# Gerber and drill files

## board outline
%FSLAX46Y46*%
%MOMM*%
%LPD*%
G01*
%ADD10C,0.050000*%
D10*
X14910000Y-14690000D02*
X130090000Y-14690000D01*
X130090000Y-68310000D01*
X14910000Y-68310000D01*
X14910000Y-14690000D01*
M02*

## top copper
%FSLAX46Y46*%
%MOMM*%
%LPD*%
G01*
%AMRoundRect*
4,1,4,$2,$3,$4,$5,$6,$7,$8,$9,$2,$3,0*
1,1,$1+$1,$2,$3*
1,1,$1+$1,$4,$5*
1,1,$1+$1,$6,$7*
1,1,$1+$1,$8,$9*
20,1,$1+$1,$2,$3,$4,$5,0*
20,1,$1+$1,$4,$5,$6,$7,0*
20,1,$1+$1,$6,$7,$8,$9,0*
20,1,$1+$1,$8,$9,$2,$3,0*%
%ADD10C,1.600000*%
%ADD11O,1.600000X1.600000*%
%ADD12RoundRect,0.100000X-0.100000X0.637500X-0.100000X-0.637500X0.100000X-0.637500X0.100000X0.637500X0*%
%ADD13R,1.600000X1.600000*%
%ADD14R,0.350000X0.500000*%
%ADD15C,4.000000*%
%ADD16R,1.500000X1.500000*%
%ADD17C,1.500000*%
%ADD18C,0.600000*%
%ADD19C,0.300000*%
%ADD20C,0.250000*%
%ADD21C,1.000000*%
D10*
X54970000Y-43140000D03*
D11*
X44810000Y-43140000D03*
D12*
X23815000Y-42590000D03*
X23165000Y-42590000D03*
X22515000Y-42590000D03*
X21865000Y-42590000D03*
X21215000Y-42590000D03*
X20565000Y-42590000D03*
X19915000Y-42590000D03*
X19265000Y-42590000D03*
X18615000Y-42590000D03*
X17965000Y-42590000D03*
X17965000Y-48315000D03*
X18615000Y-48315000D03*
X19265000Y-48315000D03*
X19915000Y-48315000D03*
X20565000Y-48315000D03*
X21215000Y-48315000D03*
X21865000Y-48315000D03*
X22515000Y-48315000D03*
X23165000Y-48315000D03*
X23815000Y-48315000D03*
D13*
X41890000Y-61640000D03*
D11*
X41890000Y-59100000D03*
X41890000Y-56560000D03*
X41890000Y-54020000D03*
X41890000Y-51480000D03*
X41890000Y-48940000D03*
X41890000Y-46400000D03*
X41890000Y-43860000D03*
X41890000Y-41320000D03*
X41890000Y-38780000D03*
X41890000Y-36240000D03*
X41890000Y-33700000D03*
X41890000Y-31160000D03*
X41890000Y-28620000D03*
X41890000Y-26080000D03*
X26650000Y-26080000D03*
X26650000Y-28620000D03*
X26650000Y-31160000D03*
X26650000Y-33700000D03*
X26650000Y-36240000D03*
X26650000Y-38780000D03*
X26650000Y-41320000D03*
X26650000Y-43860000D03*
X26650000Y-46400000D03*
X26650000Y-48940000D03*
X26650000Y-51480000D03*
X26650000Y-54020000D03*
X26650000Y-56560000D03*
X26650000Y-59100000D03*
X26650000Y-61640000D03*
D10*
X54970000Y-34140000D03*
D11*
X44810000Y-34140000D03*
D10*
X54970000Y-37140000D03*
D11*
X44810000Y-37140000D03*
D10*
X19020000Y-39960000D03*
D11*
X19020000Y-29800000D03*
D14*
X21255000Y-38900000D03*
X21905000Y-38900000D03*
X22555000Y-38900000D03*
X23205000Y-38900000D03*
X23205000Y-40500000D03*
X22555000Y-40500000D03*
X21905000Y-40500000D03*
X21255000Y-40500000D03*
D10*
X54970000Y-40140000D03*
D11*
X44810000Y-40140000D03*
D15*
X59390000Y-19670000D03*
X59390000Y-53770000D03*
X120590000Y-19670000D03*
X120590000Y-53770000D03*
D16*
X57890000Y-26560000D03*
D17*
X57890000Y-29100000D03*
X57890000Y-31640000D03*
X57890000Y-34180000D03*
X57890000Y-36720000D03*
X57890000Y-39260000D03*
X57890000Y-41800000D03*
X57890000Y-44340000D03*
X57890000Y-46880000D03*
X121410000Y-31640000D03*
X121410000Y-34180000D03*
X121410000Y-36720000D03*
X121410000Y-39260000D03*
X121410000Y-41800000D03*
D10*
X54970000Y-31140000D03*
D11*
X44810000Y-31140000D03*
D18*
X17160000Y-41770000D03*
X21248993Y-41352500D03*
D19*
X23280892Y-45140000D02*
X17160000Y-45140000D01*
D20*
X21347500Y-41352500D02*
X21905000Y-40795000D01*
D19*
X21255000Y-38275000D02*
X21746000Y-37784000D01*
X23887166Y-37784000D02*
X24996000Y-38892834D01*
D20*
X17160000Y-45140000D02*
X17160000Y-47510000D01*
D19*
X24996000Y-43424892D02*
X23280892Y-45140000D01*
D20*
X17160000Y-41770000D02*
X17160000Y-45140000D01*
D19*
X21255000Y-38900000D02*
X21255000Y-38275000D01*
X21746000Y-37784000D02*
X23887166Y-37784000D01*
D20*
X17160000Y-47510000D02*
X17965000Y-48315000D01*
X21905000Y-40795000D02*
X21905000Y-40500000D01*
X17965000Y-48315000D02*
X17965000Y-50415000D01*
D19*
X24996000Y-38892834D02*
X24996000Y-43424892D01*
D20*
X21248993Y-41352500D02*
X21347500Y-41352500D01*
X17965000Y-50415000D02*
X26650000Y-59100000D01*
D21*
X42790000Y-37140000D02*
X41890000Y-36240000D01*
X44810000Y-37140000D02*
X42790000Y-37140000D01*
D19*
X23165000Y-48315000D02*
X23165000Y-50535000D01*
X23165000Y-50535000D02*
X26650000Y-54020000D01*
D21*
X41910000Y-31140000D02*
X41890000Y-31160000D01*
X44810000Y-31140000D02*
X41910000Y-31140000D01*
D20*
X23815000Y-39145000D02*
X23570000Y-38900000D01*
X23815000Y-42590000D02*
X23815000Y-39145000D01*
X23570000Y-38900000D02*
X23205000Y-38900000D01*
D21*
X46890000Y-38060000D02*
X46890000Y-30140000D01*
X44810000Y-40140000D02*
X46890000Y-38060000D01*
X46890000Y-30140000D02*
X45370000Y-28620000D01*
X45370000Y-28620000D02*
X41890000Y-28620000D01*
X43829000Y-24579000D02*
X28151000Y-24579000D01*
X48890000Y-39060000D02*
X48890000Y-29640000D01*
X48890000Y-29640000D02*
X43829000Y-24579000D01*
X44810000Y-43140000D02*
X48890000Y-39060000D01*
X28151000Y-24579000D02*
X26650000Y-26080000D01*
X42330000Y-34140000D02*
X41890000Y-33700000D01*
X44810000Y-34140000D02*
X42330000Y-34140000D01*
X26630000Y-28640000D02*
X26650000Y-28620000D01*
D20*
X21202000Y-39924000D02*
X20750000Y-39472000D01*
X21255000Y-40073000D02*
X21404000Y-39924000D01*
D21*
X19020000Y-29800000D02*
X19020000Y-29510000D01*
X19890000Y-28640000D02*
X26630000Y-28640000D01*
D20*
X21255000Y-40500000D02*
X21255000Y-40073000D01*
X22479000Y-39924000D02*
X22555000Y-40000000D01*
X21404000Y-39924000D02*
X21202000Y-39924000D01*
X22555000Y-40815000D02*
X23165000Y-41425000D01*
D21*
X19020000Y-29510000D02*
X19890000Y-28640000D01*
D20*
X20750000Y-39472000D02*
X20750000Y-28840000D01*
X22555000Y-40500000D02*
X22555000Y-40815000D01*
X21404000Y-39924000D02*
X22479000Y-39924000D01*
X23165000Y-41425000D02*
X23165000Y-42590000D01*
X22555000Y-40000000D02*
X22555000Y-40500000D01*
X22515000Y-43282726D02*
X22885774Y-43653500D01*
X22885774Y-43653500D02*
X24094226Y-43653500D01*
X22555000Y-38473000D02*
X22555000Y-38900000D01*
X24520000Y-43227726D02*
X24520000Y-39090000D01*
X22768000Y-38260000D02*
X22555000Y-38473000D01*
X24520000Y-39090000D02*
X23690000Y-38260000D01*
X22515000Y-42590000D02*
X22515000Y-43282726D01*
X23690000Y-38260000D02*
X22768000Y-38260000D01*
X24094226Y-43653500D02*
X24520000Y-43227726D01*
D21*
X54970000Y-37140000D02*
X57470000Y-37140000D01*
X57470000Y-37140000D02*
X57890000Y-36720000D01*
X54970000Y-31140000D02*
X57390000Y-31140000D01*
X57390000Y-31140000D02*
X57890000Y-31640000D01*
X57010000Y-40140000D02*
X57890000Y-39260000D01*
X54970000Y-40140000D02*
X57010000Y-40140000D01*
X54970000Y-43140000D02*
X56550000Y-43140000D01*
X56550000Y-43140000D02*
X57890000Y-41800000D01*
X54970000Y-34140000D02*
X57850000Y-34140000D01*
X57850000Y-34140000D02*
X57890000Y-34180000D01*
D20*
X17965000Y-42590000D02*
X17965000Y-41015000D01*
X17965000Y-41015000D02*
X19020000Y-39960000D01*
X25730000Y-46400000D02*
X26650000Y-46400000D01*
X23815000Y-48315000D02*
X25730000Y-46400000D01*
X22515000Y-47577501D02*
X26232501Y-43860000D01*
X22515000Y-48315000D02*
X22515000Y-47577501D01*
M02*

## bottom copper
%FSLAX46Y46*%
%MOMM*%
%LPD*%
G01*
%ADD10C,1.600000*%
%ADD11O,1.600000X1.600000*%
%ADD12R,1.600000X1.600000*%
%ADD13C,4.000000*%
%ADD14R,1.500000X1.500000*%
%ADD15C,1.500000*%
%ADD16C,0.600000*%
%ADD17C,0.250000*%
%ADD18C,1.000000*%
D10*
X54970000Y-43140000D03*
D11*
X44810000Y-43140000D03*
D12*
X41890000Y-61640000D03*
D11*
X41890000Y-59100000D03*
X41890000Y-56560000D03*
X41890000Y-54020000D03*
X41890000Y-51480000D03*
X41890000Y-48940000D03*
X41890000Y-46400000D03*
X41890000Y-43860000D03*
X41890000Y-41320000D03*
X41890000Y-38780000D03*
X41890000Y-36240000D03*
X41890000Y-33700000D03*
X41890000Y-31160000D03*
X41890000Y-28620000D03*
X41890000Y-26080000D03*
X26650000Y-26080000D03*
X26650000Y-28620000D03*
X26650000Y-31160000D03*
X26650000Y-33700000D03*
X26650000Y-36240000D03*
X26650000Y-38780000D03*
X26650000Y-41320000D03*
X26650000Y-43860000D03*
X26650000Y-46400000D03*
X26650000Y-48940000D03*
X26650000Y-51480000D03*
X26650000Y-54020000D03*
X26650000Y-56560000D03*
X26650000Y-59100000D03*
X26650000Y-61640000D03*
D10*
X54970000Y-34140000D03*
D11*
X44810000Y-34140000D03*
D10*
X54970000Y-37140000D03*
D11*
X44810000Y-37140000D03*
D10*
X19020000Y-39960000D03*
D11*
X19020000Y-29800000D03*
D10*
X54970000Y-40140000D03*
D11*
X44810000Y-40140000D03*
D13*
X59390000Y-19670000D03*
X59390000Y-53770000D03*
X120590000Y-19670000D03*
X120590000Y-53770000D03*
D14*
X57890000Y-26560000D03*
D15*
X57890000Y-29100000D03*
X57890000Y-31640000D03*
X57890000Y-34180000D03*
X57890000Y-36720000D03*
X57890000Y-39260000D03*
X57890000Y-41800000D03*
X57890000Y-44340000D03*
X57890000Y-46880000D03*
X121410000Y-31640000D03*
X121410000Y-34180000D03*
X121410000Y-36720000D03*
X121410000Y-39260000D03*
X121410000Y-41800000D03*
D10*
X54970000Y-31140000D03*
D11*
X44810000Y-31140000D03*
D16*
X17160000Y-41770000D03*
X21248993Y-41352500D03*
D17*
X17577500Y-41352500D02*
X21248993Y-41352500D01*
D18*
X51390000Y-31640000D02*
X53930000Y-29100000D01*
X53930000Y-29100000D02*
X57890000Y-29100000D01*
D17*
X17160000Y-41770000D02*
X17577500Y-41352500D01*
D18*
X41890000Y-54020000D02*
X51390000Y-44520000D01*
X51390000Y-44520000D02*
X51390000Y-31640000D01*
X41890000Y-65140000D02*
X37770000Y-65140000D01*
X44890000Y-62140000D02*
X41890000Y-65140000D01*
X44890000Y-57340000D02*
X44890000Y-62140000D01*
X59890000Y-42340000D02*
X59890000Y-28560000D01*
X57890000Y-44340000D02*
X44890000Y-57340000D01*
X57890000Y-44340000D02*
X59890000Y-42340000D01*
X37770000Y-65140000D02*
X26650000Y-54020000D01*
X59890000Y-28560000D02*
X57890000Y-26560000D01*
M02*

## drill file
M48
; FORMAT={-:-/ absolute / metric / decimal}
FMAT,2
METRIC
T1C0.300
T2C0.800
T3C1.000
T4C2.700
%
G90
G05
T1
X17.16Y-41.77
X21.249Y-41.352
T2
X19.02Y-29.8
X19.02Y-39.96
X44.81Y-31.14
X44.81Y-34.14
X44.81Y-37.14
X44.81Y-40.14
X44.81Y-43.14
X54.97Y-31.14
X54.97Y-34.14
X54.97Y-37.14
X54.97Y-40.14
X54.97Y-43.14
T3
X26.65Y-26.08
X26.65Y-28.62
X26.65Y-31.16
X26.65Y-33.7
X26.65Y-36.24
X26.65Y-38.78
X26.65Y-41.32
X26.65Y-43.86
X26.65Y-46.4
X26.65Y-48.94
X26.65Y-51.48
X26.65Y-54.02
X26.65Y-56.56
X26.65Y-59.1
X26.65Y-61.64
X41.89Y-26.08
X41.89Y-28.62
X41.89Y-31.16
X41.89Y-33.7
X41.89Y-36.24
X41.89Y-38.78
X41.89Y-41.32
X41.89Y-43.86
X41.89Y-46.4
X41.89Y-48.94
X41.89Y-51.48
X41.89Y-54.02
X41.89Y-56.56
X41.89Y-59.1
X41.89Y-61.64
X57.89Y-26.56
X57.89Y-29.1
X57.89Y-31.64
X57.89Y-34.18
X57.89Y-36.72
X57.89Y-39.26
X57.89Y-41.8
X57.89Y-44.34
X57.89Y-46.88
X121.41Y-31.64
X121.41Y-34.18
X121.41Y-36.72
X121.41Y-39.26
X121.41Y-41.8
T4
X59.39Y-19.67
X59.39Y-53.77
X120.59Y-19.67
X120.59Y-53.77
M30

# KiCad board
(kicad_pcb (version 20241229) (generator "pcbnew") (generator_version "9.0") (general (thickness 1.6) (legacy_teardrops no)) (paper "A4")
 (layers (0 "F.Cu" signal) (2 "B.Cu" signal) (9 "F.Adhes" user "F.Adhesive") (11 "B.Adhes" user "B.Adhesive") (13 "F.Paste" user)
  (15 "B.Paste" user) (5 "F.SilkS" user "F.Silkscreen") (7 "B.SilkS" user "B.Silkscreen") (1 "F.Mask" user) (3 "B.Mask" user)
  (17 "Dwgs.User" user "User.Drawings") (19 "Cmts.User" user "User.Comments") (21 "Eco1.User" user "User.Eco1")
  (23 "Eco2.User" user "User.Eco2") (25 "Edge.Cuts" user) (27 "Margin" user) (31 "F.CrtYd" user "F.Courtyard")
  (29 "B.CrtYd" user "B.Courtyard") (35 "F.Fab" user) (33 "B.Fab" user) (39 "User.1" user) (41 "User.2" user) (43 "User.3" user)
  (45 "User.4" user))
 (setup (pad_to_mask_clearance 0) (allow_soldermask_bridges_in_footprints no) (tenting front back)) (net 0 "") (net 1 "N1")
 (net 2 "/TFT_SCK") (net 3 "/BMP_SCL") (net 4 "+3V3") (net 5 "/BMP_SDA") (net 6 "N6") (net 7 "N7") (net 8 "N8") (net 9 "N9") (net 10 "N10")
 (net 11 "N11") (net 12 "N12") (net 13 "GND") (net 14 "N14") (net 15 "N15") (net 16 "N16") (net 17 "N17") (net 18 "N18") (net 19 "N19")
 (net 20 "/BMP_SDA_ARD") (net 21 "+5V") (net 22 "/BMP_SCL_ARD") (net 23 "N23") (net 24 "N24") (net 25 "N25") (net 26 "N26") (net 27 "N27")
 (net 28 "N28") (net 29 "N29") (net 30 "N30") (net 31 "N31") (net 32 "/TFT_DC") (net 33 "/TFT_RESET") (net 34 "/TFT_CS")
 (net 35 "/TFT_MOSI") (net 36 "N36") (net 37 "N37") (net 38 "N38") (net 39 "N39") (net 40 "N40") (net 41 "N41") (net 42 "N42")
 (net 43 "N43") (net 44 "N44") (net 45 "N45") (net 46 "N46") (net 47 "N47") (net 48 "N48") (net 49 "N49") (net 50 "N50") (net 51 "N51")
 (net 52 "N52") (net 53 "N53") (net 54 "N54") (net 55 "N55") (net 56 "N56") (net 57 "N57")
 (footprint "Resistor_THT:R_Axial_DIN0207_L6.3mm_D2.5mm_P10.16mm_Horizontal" (layer "F.Cu") (at 54.97 43.14 180)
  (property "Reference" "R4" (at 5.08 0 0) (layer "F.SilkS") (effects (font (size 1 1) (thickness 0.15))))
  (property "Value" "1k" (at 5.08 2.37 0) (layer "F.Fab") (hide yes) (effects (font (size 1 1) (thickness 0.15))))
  (pad "1" thru_hole circle (at 0 0 180) (size 1.6 1.6) (drill 0.8) (layers "*.Cu" "*.Mask") (remove_unused_layers no) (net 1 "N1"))
  (pad "2" thru_hole oval (at 10.16 0 180) (size 1.6 1.6) (drill 0.8) (layers "*.Cu" "*.Mask") (remove_unused_layers no) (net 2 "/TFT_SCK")))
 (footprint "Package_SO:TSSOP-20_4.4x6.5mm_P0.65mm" (layer "F.Cu") (at 20.89 45.4525 -90)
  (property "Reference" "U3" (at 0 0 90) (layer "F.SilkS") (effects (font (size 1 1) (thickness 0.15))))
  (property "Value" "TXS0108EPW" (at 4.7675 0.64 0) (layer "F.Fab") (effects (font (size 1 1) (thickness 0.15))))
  (pad "1" smd roundrect (at -2.8625 -2.925 270) (size 1.475 0.4) (layers "F.Cu" "F.Mask" "F.Paste") (roundrect_rratio 0.25)
   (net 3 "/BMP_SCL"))
  (pad "2" smd roundrect (at -2.8625 -2.275 270) (size 1.475 0.4) (layers "F.Cu" "F.Mask" "F.Paste") (roundrect_rratio 0.25) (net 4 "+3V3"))
  (pad "3" smd roundrect (at -2.8625 -1.625 270) (size 1.475 0.4) (layers "F.Cu" "F.Mask" "F.Paste") (roundrect_rratio 0.25)
   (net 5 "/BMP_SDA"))
  (pad "4" smd roundrect (at -2.8625 -0.975 270) (size 1.475 0.4) (layers "F.Cu" "F.Mask" "F.Paste") (roundrect_rratio 0.25) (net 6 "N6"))
  (pad "5" smd roundrect (at -2.8625 -0.325 270) (size 1.475 0.4) (layers "F.Cu" "F.Mask" "F.Paste") (roundrect_rratio 0.25) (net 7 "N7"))
  (pad "6" smd roundrect (at -2.8625 0.325 270) (size 1.475 0.4) (layers "F.Cu" "F.Mask" "F.Paste") (roundrect_rratio 0.25) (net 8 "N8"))
  (pad "7" smd roundrect (at -2.8625 0.975 270) (size 1.475 0.4) (layers "F.Cu" "F.Mask" "F.Paste") (roundrect_rratio 0.25) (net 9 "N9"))
  (pad "8" smd roundrect (at -2.8625 1.625 270) (size 1.475 0.4) (layers "F.Cu" "F.Mask" "F.Paste") (roundrect_rratio 0.25) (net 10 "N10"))
  (pad "9" smd roundrect (at -2.8625 2.275 270) (size 1.475 0.4) (layers "F.Cu" "F.Mask" "F.Paste") (roundrect_rratio 0.25) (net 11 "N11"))
  (pad "10" smd roundrect (at -2.8625 2.925 270) (size 1.475 0.4) (layers "F.Cu" "F.Mask" "F.Paste") (roundrect_rratio 0.25) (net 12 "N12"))
  (pad "11" smd roundrect (at 2.8625 2.925 270) (size 1.475 0.4) (layers "F.Cu" "F.Mask" "F.Paste") (roundrect_rratio 0.25) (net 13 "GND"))
  (pad "12" smd roundrect (at 2.8625 2.275 270) (size 1.475 0.4) (layers "F.Cu" "F.Mask" "F.Paste") (roundrect_rratio 0.25) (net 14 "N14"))
  (pad "13" smd roundrect (at 2.8625 1.625 270) (size 1.475 0.4) (layers "F.Cu" "F.Mask" "F.Paste") (roundrect_rratio 0.25) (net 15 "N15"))
  (pad "14" smd roundrect (at 2.8625 0.975 270) (size 1.475 0.4) (layers "F.Cu" "F.Mask" "F.Paste") (roundrect_rratio 0.25) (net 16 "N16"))
  (pad "15" smd roundrect (at 2.8625 0.325 270) (size 1.475 0.4) (layers "F.Cu" "F.Mask" "F.Paste") (roundrect_rratio 0.25) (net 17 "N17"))
  (pad "16" smd roundrect (at 2.8625 -0.325 270) (size 1.475 0.4) (layers "F.Cu" "F.Mask" "F.Paste") (roundrect_rratio 0.25) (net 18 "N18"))
  (pad "17" smd roundrect (at 2.8625 -0.975 270) (size 1.475 0.4) (layers "F.Cu" "F.Mask" "F.Paste") (roundrect_rratio 0.25) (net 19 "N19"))
  (pad "18" smd roundrect (at 2.8625 -1.625 270) (size 1.475 0.4) (layers "F.Cu" "F.Mask" "F.Paste") (roundrect_rratio 0.25)
   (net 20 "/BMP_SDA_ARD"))
  (pad "19" smd roundrect (at 2.8625 -2.275 270) (size 1.475 0.4) (layers "F.Cu" "F.Mask" "F.Paste") (roundrect_rratio 0.25) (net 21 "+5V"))
  (pad "20" smd roundrect (at 2.8625 -2.925 270) (size 1.475 0.4) (layers "F.Cu" "F.Mask" "F.Paste") (roundrect_rratio 0.25)
   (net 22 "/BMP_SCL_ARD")))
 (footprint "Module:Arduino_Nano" (layer "F.Cu") (at 41.89 61.64 180)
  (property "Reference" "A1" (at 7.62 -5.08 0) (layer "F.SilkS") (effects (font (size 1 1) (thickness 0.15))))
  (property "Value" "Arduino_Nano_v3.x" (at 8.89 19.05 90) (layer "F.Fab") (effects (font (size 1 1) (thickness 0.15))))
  (pad "1" thru_hole rect (at 0 0 180) (size 1.6 1.6) (drill 1) (layers "*.Cu" "*.Mask") (remove_unused_layers no) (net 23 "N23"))
  (pad "2" thru_hole oval (at 0 2.54 180) (size 1.6 1.6) (drill 1) (layers "*.Cu" "*.Mask") (remove_unused_layers no) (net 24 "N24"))
  (pad "3" thru_hole oval (at 0 5.08 180) (size 1.6 1.6) (drill 1) (layers "*.Cu" "*.Mask") (remove_unused_layers no) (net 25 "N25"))
  (pad "4" thru_hole oval (at 0 7.62 180) (size 1.6 1.6) (drill 1) (layers "*.Cu" "*.Mask") (remove_unused_layers no) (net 13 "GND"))
  (pad "5" thru_hole oval (at 0 10.16 180) (size 1.6 1.6) (drill 1) (layers "*.Cu" "*.Mask") (remove_unused_layers no) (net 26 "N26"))
  (pad "6" thru_hole oval (at 0 12.7 180) (size 1.6 1.6) (drill 1) (layers "*.Cu" "*.Mask") (remove_unused_layers no) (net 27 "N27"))
  (pad "7" thru_hole oval (at 0 15.24 180) (size 1.6 1.6) (drill 1) (layers "*.Cu" "*.Mask") (remove_unused_layers no) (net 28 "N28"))
  (pad "8" thru_hole oval (at 0 17.78 180) (size 1.6 1.6) (drill 1) (layers "*.Cu" "*.Mask") (remove_unused_layers no) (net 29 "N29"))
  (pad "9" thru_hole oval (at 0 20.32 180) (size 1.6 1.6) (drill 1) (layers "*.Cu" "*.Mask") (remove_unused_layers no) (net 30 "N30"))
  (pad "10" thru_hole oval (at 0 22.86 180) (size 1.6 1.6) (drill 1) (layers "*.Cu" "*.Mask") (remove_unused_layers no) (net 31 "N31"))
  (pad "11" thru_hole oval (at 0 25.4 180) (size 1.6 1.6) (drill 1) (layers "*.Cu" "*.Mask") (remove_unused_layers no) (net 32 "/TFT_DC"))
  (pad "12" thru_hole oval (at 0 27.94 180) (size 1.6 1.6) (drill 1) (layers "*.Cu" "*.Mask") (remove_unused_layers no)
   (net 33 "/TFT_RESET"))
  (pad "13" thru_hole oval (at 0 30.48 180) (size 1.6 1.6) (drill 1) (layers "*.Cu" "*.Mask") (remove_unused_layers no) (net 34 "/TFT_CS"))
  (pad "14" thru_hole oval (at 0 33.02 180) (size 1.6 1.6) (drill 1) (layers "*.Cu" "*.Mask") (remove_unused_layers no) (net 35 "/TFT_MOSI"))
  (pad "15" thru_hole oval (at 0 35.56 180) (size 1.6 1.6) (drill 1) (layers "*.Cu" "*.Mask") (remove_unused_layers no) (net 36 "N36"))
  (pad "16" thru_hole oval (at 15.24 35.56 180) (size 1.6 1.6) (drill 1) (layers "*.Cu" "*.Mask") (remove_unused_layers no)
   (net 2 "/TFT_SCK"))
  (pad "17" thru_hole oval (at 15.24 33.02 180) (size 1.6 1.6) (drill 1) (layers "*.Cu" "*.Mask") (remove_unused_layers no) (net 4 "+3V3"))
  (pad "18" thru_hole oval (at 15.24 30.48 180) (size 1.6 1.6) (drill 1) (layers "*.Cu" "*.Mask") (remove_unused_layers no) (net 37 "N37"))
  (pad "19" thru_hole oval (at 15.24 27.94 180) (size 1.6 1.6) (drill 1) (layers "*.Cu" "*.Mask") (remove_unused_layers no) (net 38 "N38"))
  (pad "20" thru_hole oval (at 15.24 25.4 180) (size 1.6 1.6) (drill 1) (layers "*.Cu" "*.Mask") (remove_unused_layers no) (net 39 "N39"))
  (pad "21" thru_hole oval (at 15.24 22.86 180) (size 1.6 1.6) (drill 1) (layers "*.Cu" "*.Mask") (remove_unused_layers no) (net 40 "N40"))
  (pad "22" thru_hole oval (at 15.24 20.32 180) (size 1.6 1.6) (drill 1) (layers "*.Cu" "*.Mask") (remove_unused_layers no) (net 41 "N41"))
  (pad "23" thru_hole oval (at 15.24 17.78 180) (size 1.6 1.6) (drill 1) (layers "*.Cu" "*.Mask") (remove_unused_layers no)
   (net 20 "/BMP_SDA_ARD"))
  (pad "24" thru_hole oval (at 15.24 15.24 180) (size 1.6 1.6) (drill 1) (layers "*.Cu" "*.Mask") (remove_unused_layers no)
   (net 22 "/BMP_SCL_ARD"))
  (pad "25" thru_hole oval (at 15.24 12.7 180) (size 1.6 1.6) (drill 1) (layers "*.Cu" "*.Mask") (remove_unused_layers no) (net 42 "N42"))
  (pad "26" thru_hole oval (at 15.24 10.16 180) (size 1.6 1.6) (drill 1) (layers "*.Cu" "*.Mask") (remove_unused_layers no) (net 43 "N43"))
  (pad "27" thru_hole oval (at 15.24 7.62 180) (size 1.6 1.6) (drill 1) (layers "*.Cu" "*.Mask") (remove_unused_layers no) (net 21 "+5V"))
  (pad "28" thru_hole oval (at 15.24 5.08 180) (size 1.6 1.6) (drill 1) (layers "*.Cu" "*.Mask") (remove_unused_layers no) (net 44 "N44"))
  (pad "29" thru_hole oval (at 15.24 2.54 180) (size 1.6 1.6) (drill 1) (layers "*.Cu" "*.Mask") (remove_unused_layers no) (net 13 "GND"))
  (pad "30" thru_hole oval (at 15.24 0 180) (size 1.6 1.6) (drill 1) (layers "*.Cu" "*.Mask") (remove_unused_layers no) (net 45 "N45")))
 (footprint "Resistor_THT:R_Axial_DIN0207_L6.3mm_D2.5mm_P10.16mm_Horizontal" (layer "F.Cu") (at 54.97 34.14 180)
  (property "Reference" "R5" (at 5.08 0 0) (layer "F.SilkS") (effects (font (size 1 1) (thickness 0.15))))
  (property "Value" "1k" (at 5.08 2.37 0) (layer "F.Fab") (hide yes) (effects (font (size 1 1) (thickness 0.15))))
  (pad "1" thru_hole circle (at 0 0 180) (size 1.6 1.6) (drill 0.8) (layers "*.Cu" "*.Mask") (remove_unused_layers no) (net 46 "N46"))
  (pad "2" thru_hole oval (at 10.16 0 180) (size 1.6 1.6) (drill 0.8) (layers "*.Cu" "*.Mask") (remove_unused_layers no)
   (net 33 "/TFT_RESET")))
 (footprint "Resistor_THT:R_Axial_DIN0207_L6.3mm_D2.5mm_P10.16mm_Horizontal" (layer "F.Cu") (at 54.97 37.14 180)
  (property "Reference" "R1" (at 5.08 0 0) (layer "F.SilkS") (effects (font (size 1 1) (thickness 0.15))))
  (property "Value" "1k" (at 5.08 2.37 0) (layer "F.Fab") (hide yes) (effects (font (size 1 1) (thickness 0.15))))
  (pad "1" thru_hole circle (at 0 0 180) (size 1.6 1.6) (drill 0.8) (layers "*.Cu" "*.Mask") (remove_unused_layers no) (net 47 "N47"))
  (pad "2" thru_hole oval (at 10.16 0 180) (size 1.6 1.6) (drill 0.8) (layers "*.Cu" "*.Mask") (remove_unused_layers no) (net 32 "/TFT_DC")))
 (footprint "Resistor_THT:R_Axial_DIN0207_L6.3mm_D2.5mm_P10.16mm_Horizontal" (layer "F.Cu") (at 19.02 39.96 90)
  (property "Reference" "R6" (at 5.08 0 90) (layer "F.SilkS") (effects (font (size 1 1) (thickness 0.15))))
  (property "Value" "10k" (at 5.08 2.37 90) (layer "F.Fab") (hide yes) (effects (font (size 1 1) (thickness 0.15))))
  (pad "1" thru_hole circle (at 0 0 90) (size 1.6 1.6) (drill 0.8) (layers "*.Cu" "*.Mask") (remove_unused_layers no) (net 12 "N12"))
  (pad "2" thru_hole oval (at 10.16 0 90) (size 1.6 1.6) (drill 0.8) (layers "*.Cu" "*.Mask") (remove_unused_layers no) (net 4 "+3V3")))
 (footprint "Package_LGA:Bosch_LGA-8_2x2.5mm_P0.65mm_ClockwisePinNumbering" (layer "F.Cu") (at 22.23 39.7)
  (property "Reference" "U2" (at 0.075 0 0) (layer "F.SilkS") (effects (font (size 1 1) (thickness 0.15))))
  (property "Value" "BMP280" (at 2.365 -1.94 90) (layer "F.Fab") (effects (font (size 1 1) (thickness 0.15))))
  (pad "1" smd rect (at -0.975 -0.8 90) (size 0.5 0.35) (layers "F.Cu" "F.Mask" "F.Paste") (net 13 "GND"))
  (pad "2" smd rect (at -0.325 -0.8 90) (size 0.5 0.35) (layers "F.Cu" "F.Mask" "F.Paste") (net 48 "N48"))
  (pad "3" smd rect (at 0.325 -0.8 90) (size 0.5 0.35) (layers "F.Cu" "F.Mask" "F.Paste") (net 5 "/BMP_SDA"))
  (pad "4" smd rect (at 0.975 -0.8 90) (size 0.5 0.35) (layers "F.Cu" "F.Mask" "F.Paste") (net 3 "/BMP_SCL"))
  (pad "5" smd rect (at 0.975 0.8 90) (size 0.5 0.35) (layers "F.Cu" "F.Mask" "F.Paste") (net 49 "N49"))
  (pad "6" smd rect (at 0.325 0.8 90) (size 0.5 0.35) (layers "F.Cu" "F.Mask" "F.Paste") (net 4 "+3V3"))
  (pad "7" smd rect (at -0.325 0.8 90) (size 0.5 0.35) (layers "F.Cu" "F.Mask" "F.Paste") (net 13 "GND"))
  (pad "8" smd rect (at -0.975 0.8 90) (size 0.5 0.35) (layers "F.Cu" "F.Mask" "F.Paste") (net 4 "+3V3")))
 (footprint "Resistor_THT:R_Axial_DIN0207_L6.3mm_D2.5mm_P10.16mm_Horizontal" (layer "F.Cu") (at 54.97 40.14 180)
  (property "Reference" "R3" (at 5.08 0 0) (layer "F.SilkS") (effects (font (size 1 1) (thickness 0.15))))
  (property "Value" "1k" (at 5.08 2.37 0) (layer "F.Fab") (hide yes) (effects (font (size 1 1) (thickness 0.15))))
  (pad "1" thru_hole circle (at 0 0 180) (size 1.6 1.6) (drill 0.8) (layers "*.Cu" "*.Mask") (remove_unused_layers no) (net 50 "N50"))
  (pad "2" thru_hole oval (at 10.16 0 180) (size 1.6 1.6) (drill 0.8) (layers "*.Cu" "*.Mask") (remove_unused_layers no)
   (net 35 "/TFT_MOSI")))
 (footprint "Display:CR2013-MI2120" (layer "F.Cu") (at 57.89 26.56)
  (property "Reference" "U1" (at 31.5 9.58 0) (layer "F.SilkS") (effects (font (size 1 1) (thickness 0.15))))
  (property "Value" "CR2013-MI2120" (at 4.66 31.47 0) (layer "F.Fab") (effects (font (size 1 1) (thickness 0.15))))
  (pad "" thru_hole circle (at 1.5 -6.89) (size 4 4) (drill 2.7) (layers "*.Cu" "*.Mask") (remove_unused_layers no))
  (pad "" thru_hole circle (at 1.5 27.21) (size 4 4) (drill 2.7) (layers "*.Cu" "*.Mask") (remove_unused_layers no))
  (pad "" thru_hole circle (at 62.7 -6.89) (size 4 4) (drill 2.7) (layers "*.Cu" "*.Mask") (remove_unused_layers no))
  (pad "" thru_hole circle (at 62.7 27.21) (size 4 4) (drill 2.7) (layers "*.Cu" "*.Mask") (remove_unused_layers no))
  (pad "1" thru_hole rect (at 0 0) (size 1.5 1.5) (drill 1) (layers "*.Cu" "*.Mask") (remove_unused_layers no) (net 21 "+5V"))
  (pad "2" thru_hole circle (at 0 2.54) (size 1.5 1.5) (drill 1) (layers "*.Cu" "*.Mask") (remove_unused_layers no) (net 13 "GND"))
  (pad "3" thru_hole circle (at 0 5.08) (size 1.5 1.5) (drill 1) (layers "*.Cu" "*.Mask") (remove_unused_layers no) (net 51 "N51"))
  (pad "4" thru_hole circle (at 0 7.62) (size 1.5 1.5) (drill 1) (layers "*.Cu" "*.Mask") (remove_unused_layers no) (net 46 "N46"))
  (pad "5" thru_hole circle (at 0 10.16) (size 1.5 1.5) (drill 1) (layers "*.Cu" "*.Mask") (remove_unused_layers no) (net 47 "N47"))
  (pad "6" thru_hole circle (at 0 12.7) (size 1.5 1.5) (drill 1) (layers "*.Cu" "*.Mask") (remove_unused_layers no) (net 50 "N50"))
  (pad "7" thru_hole circle (at 0 15.24) (size 1.5 1.5) (drill 1) (layers "*.Cu" "*.Mask") (remove_unused_layers no) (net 1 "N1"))
  (pad "8" thru_hole circle (at 0 17.78) (size 1.5 1.5) (drill 1) (layers "*.Cu" "*.Mask") (remove_unused_layers no) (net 21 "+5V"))
  (pad "9" thru_hole circle (at 0 20.32) (size 1.5 1.5) (drill 1) (layers "*.Cu" "*.Mask") (remove_unused_layers no) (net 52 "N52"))
  (pad "10" thru_hole circle (at 63.52 5.08) (size 1.5 1.5) (drill 1) (layers "*.Cu" "*.Mask") (remove_unused_layers no) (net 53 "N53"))
  (pad "11" thru_hole circle (at 63.52 7.62) (size 1.5 1.5) (drill 1) (layers "*.Cu" "*.Mask") (remove_unused_layers no) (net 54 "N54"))
  (pad "12" thru_hole circle (at 63.52 10.16) (size 1.5 1.5) (drill 1) (layers "*.Cu" "*.Mask") (remove_unused_layers no) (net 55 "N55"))
  (pad "13" thru_hole circle (at 63.52 12.7) (size 1.5 1.5) (drill 1) (layers "*.Cu" "*.Mask") (remove_unused_layers no) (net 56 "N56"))
  (pad "14" thru_hole circle (at 63.52 15.24) (size 1.5 1.5) (drill 1) (layers "*.Cu" "*.Mask") (remove_unused_layers no) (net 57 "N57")))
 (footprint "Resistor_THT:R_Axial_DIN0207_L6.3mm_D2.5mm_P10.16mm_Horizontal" (layer "F.Cu") (at 54.97 31.14 180)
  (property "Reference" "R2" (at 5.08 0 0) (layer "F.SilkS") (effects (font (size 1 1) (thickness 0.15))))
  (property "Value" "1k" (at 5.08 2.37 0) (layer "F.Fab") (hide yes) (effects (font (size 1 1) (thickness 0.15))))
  (pad "1" thru_hole circle (at 0 0 180) (size 1.6 1.6) (drill 0.8) (layers "*.Cu" "*.Mask") (remove_unused_layers no) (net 51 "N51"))
  (pad "2" thru_hole oval (at 10.16 0 180) (size 1.6 1.6) (drill 0.8) (layers "*.Cu" "*.Mask") (remove_unused_layers no) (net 34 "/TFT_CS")))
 (gr_rect (start 14.91 14.69) (end 130.09 68.31) (stroke (width 0.05) (type default)) (fill no) (layer "Edge.Cuts"))
 (segment (start 23.280892 45.14) (end 17.16 45.14) (width 0.3) (layer "F.Cu") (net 13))
 (segment (start 21.3475 41.3525) (end 21.905 40.795) (width 0.25) (layer "F.Cu") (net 13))
 (segment (start 21.255 38.275) (end 21.746 37.784) (width 0.3) (layer "F.Cu") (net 13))
 (segment (start 23.887166 37.784) (end 24.996 38.892834) (width 0.3) (layer "F.Cu") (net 13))
 (segment (start 17.16 45.14) (end 17.16 47.51) (width 0.25) (layer "F.Cu") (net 13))
 (segment (start 24.996 43.424892) (end 23.280892 45.14) (width 0.3) (layer "F.Cu") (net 13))
 (segment (start 17.16 41.77) (end 17.16 45.14) (width 0.25) (layer "F.Cu") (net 13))
 (segment (start 21.255 38.9) (end 21.255 38.275) (width 0.3) (layer "F.Cu") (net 13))
 (segment (start 21.746 37.784) (end 23.887166 37.784) (width 0.3) (layer "F.Cu") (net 13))
 (segment (start 17.16 47.51) (end 17.965 48.315) (width 0.25) (layer "F.Cu") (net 13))
 (segment (start 21.905 40.795) (end 21.905 40.5) (width 0.25) (layer "F.Cu") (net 13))
 (segment (start 17.965 48.315) (end 17.965 50.415) (width 0.25) (layer "F.Cu") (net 13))
 (segment (start 24.996 38.892834) (end 24.996 43.424892) (width 0.3) (layer "F.Cu") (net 13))
 (segment (start 21.248993 41.3525) (end 21.3475 41.3525) (width 0.25) (layer "F.Cu") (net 13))
 (segment (start 17.965 50.415) (end 26.65 59.1) (width 0.25) (layer "F.Cu") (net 13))
 (via (at 17.16 41.77) (size 0.6) (drill 0.3) (layers "F.Cu" "B.Cu") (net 13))
 (via (at 21.248993 41.3525) (size 0.6) (drill 0.3) (layers "F.Cu" "B.Cu") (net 13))
 (segment (start 17.5775 41.3525) (end 21.248993 41.3525) (width 0.25) (layer "B.Cu") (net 13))
 (segment (start 51.39 31.64) (end 53.93 29.1) (width 1) (layer "B.Cu") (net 13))
 (segment (start 53.93 29.1) (end 57.89 29.1) (width 1) (layer "B.Cu") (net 13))
 (segment (start 17.16 41.77) (end 17.5775 41.3525) (width 0.25) (layer "B.Cu") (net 13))
 (segment (start 41.89 54.02) (end 51.39 44.52) (width 1) (layer "B.Cu") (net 13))
 (segment (start 51.39 44.52) (end 51.39 31.64) (width 1) (layer "B.Cu") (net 13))
 (segment (start 42.79 37.14) (end 41.89 36.24) (width 1) (layer "F.Cu") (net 32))
 (segment (start 44.81 37.14) (end 42.79 37.14) (width 1) (layer "F.Cu") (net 32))
 (segment (start 23.165 48.315) (end 23.165 50.535) (width 0.3) (layer "F.Cu") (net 21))
 (segment (start 23.165 50.535) (end 26.65 54.02) (width 0.3) (layer "F.Cu") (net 21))
 (segment (start 41.89 65.14) (end 37.77 65.14) (width 1) (layer "B.Cu") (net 21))
 (segment (start 44.89 62.14) (end 41.89 65.14) (width 1) (layer "B.Cu") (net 21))
 (segment (start 44.89 57.34) (end 44.89 62.14) (width 1) (layer "B.Cu") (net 21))
 (segment (start 59.89 42.34) (end 59.89 28.56) (width 1) (layer "B.Cu") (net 21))
 (segment (start 57.89 44.34) (end 44.89 57.34) (width 1) (layer "B.Cu") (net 21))
 (segment (start 57.89 44.34) (end 59.89 42.34) (width 1) (layer "B.Cu") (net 21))
 (segment (start 37.77 65.14) (end 26.65 54.02) (width 1) (layer "B.Cu") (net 21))
 (segment (start 59.89 28.56) (end 57.89 26.56) (width 1) (layer "B.Cu") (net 21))
 (segment (start 41.91 31.14) (end 41.89 31.16) (width 1) (layer "F.Cu") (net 34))
 (segment (start 44.81 31.14) (end 41.91 31.14) (width 1) (layer "F.Cu") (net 34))
 (segment (start 23.815 39.145) (end 23.57 38.9) (width 0.25) (layer "F.Cu") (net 3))
 (segment (start 23.815 42.59) (end 23.815 39.145) (width 0.25) (layer "F.Cu") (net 3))
 (segment (start 23.57 38.9) (end 23.205 38.9) (width 0.25) (layer "F.Cu") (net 3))
 (segment (start 46.89 38.06) (end 46.89 30.14) (width 1) (layer "F.Cu") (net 35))
 (segment (start 44.81 40.14) (end 46.89 38.06) (width 1) (layer "F.Cu") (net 35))
 (segment (start 46.89 30.14) (end 45.37 28.62) (width 1) (layer "F.Cu") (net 35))
 (segment (start 45.37 28.62) (end 41.89 28.62) (width 1) (layer "F.Cu") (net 35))
 (segment (start 43.829 24.579) (end 28.151 24.579) (width 1) (layer "F.Cu") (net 2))
 (segment (start 48.89 39.06) (end 48.89 29.64) (width 1) (layer "F.Cu") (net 2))
 (segment (start 48.89 29.64) (end 43.829 24.579) (width 1) (layer "F.Cu") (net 2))
 (segment (start 44.81 43.14) (end 48.89 39.06) (width 1) (layer "F.Cu") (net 2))
 (segment (start 28.151 24.579) (end 26.65 26.08) (width 1) (layer "F.Cu") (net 2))
 (segment (start 42.33 34.14) (end 41.89 33.7) (width 1) (layer "F.Cu") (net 33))
 (segment (start 44.81 34.14) (end 42.33 34.14) (width 1) (layer "F.Cu") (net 33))
 (segment (start 26.63 28.64) (end 26.65 28.62) (width 1) (layer "F.Cu") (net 4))
 (segment (start 21.202 39.924) (end 20.75 39.472) (width 0.25) (layer "F.Cu") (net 4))
 (segment (start 21.255 40.073) (end 21.404 39.924) (width 0.25) (layer "F.Cu") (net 4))
 (segment (start 19.02 29.8) (end 19.02 29.51) (width 1) (layer "F.Cu") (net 4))
 (segment (start 19.89 28.64) (end 26.63 28.64) (width 1) (layer "F.Cu") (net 4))
 (segment (start 21.255 40.5) (end 21.255 40.073) (width 0.25) (layer "F.Cu") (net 4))
 (segment (start 22.479 39.924) (end 22.555 40) (width 0.25) (layer "F.Cu") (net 4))
 (segment (start 21.404 39.924) (end 21.202 39.924) (width 0.25) (layer "F.Cu") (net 4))
 (segment (start 22.555 40.815) (end 23.165 41.425) (width 0.25) (layer "F.Cu") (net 4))
 (segment (start 19.02 29.51) (end 19.89 28.64) (width 1) (layer "F.Cu") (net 4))
 (segment (start 20.75 39.472) (end 20.75 28.84) (width 0.25) (layer "F.Cu") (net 4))
 (segment (start 22.555 40.5) (end 22.555 40.815) (width 0.25) (layer "F.Cu") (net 4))
 (segment (start 21.404 39.924) (end 22.479 39.924) (width 0.25) (layer "F.Cu") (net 4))
 (segment (start 23.165 41.425) (end 23.165 42.59) (width 0.25) (layer "F.Cu") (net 4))
 (segment (start 22.555 40) (end 22.555 40.5) (width 0.25) (layer "F.Cu") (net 4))
 (segment (start 22.515 43.282726) (end 22.885774 43.6535) (width 0.25) (layer "F.Cu") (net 5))
 (segment (start 22.885774 43.6535) (end 24.094226 43.6535) (width 0.25) (layer "F.Cu") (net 5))
 (segment (start 22.555 38.473) (end 22.555 38.9) (width 0.25) (layer "F.Cu") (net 5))
 (segment (start 24.52 43.227726) (end 24.52 39.09) (width 0.25) (layer "F.Cu") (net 5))
 (segment (start 22.768 38.26) (end 22.555 38.473) (width 0.25) (layer "F.Cu") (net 5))
 (segment (start 24.52 39.09) (end 23.69 38.26) (width 0.25) (layer "F.Cu") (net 5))
 (segment (start 22.515 42.59) (end 22.515 43.282726) (width 0.25) (layer "F.Cu") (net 5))
 (segment (start 23.69 38.26) (end 22.768 38.26) (width 0.25) (layer "F.Cu") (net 5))
 (segment (start 24.094226 43.6535) (end 24.52 43.227726) (width 0.25) (layer "F.Cu") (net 5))
 (segment (start 54.97 37.14) (end 57.47 37.14) (width 1) (layer "F.Cu") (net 47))
 (segment (start 57.47 37.14) (end 57.89 36.72) (width 1) (layer "F.Cu") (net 47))
 (segment (start 54.97 31.14) (end 57.39 31.14) (width 1) (layer "F.Cu") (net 51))
 (segment (start 57.39 31.14) (end 57.89 31.64) (width 1) (layer "F.Cu") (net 51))
 (segment (start 57.01 40.14) (end 57.89 39.26) (width 1) (layer "F.Cu") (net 50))
 (segment (start 54.97 40.14) (end 57.01 40.14) (width 1) (layer "F.Cu") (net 50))
 (segment (start 54.97 43.14) (end 56.55 43.14) (width 1) (layer "F.Cu") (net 1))
 (segment (start 56.55 43.14) (end 57.89 41.8) (width 1) (layer "F.Cu") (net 1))
 (segment (start 54.97 34.14) (end 57.85 34.14) (width 1) (layer "F.Cu") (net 46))
 (segment (start 57.85 34.14) (end 57.89 34.18) (width 1) (layer "F.Cu") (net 46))
 (segment (start 17.965 42.59) (end 17.965 41.015) (width 0.25) (layer "F.Cu") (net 12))
 (segment (start 17.965 41.015) (end 19.02 39.96) (width 0.25) (layer "F.Cu") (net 12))
 (segment (start 25.73 46.4) (end 26.65 46.4) (width 0.25) (layer "F.Cu") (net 22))
 (segment (start 23.815 48.315) (end 25.73 46.4) (width 0.25) (layer "F.Cu") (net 22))
 (segment (start 22.515 47.577501) (end 26.232501 43.86) (width 0.25) (layer "F.Cu") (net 20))
 (segment (start 22.515 48.315) (end 22.515 47.577501) (width 0.25) (layer "F.Cu") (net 20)))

